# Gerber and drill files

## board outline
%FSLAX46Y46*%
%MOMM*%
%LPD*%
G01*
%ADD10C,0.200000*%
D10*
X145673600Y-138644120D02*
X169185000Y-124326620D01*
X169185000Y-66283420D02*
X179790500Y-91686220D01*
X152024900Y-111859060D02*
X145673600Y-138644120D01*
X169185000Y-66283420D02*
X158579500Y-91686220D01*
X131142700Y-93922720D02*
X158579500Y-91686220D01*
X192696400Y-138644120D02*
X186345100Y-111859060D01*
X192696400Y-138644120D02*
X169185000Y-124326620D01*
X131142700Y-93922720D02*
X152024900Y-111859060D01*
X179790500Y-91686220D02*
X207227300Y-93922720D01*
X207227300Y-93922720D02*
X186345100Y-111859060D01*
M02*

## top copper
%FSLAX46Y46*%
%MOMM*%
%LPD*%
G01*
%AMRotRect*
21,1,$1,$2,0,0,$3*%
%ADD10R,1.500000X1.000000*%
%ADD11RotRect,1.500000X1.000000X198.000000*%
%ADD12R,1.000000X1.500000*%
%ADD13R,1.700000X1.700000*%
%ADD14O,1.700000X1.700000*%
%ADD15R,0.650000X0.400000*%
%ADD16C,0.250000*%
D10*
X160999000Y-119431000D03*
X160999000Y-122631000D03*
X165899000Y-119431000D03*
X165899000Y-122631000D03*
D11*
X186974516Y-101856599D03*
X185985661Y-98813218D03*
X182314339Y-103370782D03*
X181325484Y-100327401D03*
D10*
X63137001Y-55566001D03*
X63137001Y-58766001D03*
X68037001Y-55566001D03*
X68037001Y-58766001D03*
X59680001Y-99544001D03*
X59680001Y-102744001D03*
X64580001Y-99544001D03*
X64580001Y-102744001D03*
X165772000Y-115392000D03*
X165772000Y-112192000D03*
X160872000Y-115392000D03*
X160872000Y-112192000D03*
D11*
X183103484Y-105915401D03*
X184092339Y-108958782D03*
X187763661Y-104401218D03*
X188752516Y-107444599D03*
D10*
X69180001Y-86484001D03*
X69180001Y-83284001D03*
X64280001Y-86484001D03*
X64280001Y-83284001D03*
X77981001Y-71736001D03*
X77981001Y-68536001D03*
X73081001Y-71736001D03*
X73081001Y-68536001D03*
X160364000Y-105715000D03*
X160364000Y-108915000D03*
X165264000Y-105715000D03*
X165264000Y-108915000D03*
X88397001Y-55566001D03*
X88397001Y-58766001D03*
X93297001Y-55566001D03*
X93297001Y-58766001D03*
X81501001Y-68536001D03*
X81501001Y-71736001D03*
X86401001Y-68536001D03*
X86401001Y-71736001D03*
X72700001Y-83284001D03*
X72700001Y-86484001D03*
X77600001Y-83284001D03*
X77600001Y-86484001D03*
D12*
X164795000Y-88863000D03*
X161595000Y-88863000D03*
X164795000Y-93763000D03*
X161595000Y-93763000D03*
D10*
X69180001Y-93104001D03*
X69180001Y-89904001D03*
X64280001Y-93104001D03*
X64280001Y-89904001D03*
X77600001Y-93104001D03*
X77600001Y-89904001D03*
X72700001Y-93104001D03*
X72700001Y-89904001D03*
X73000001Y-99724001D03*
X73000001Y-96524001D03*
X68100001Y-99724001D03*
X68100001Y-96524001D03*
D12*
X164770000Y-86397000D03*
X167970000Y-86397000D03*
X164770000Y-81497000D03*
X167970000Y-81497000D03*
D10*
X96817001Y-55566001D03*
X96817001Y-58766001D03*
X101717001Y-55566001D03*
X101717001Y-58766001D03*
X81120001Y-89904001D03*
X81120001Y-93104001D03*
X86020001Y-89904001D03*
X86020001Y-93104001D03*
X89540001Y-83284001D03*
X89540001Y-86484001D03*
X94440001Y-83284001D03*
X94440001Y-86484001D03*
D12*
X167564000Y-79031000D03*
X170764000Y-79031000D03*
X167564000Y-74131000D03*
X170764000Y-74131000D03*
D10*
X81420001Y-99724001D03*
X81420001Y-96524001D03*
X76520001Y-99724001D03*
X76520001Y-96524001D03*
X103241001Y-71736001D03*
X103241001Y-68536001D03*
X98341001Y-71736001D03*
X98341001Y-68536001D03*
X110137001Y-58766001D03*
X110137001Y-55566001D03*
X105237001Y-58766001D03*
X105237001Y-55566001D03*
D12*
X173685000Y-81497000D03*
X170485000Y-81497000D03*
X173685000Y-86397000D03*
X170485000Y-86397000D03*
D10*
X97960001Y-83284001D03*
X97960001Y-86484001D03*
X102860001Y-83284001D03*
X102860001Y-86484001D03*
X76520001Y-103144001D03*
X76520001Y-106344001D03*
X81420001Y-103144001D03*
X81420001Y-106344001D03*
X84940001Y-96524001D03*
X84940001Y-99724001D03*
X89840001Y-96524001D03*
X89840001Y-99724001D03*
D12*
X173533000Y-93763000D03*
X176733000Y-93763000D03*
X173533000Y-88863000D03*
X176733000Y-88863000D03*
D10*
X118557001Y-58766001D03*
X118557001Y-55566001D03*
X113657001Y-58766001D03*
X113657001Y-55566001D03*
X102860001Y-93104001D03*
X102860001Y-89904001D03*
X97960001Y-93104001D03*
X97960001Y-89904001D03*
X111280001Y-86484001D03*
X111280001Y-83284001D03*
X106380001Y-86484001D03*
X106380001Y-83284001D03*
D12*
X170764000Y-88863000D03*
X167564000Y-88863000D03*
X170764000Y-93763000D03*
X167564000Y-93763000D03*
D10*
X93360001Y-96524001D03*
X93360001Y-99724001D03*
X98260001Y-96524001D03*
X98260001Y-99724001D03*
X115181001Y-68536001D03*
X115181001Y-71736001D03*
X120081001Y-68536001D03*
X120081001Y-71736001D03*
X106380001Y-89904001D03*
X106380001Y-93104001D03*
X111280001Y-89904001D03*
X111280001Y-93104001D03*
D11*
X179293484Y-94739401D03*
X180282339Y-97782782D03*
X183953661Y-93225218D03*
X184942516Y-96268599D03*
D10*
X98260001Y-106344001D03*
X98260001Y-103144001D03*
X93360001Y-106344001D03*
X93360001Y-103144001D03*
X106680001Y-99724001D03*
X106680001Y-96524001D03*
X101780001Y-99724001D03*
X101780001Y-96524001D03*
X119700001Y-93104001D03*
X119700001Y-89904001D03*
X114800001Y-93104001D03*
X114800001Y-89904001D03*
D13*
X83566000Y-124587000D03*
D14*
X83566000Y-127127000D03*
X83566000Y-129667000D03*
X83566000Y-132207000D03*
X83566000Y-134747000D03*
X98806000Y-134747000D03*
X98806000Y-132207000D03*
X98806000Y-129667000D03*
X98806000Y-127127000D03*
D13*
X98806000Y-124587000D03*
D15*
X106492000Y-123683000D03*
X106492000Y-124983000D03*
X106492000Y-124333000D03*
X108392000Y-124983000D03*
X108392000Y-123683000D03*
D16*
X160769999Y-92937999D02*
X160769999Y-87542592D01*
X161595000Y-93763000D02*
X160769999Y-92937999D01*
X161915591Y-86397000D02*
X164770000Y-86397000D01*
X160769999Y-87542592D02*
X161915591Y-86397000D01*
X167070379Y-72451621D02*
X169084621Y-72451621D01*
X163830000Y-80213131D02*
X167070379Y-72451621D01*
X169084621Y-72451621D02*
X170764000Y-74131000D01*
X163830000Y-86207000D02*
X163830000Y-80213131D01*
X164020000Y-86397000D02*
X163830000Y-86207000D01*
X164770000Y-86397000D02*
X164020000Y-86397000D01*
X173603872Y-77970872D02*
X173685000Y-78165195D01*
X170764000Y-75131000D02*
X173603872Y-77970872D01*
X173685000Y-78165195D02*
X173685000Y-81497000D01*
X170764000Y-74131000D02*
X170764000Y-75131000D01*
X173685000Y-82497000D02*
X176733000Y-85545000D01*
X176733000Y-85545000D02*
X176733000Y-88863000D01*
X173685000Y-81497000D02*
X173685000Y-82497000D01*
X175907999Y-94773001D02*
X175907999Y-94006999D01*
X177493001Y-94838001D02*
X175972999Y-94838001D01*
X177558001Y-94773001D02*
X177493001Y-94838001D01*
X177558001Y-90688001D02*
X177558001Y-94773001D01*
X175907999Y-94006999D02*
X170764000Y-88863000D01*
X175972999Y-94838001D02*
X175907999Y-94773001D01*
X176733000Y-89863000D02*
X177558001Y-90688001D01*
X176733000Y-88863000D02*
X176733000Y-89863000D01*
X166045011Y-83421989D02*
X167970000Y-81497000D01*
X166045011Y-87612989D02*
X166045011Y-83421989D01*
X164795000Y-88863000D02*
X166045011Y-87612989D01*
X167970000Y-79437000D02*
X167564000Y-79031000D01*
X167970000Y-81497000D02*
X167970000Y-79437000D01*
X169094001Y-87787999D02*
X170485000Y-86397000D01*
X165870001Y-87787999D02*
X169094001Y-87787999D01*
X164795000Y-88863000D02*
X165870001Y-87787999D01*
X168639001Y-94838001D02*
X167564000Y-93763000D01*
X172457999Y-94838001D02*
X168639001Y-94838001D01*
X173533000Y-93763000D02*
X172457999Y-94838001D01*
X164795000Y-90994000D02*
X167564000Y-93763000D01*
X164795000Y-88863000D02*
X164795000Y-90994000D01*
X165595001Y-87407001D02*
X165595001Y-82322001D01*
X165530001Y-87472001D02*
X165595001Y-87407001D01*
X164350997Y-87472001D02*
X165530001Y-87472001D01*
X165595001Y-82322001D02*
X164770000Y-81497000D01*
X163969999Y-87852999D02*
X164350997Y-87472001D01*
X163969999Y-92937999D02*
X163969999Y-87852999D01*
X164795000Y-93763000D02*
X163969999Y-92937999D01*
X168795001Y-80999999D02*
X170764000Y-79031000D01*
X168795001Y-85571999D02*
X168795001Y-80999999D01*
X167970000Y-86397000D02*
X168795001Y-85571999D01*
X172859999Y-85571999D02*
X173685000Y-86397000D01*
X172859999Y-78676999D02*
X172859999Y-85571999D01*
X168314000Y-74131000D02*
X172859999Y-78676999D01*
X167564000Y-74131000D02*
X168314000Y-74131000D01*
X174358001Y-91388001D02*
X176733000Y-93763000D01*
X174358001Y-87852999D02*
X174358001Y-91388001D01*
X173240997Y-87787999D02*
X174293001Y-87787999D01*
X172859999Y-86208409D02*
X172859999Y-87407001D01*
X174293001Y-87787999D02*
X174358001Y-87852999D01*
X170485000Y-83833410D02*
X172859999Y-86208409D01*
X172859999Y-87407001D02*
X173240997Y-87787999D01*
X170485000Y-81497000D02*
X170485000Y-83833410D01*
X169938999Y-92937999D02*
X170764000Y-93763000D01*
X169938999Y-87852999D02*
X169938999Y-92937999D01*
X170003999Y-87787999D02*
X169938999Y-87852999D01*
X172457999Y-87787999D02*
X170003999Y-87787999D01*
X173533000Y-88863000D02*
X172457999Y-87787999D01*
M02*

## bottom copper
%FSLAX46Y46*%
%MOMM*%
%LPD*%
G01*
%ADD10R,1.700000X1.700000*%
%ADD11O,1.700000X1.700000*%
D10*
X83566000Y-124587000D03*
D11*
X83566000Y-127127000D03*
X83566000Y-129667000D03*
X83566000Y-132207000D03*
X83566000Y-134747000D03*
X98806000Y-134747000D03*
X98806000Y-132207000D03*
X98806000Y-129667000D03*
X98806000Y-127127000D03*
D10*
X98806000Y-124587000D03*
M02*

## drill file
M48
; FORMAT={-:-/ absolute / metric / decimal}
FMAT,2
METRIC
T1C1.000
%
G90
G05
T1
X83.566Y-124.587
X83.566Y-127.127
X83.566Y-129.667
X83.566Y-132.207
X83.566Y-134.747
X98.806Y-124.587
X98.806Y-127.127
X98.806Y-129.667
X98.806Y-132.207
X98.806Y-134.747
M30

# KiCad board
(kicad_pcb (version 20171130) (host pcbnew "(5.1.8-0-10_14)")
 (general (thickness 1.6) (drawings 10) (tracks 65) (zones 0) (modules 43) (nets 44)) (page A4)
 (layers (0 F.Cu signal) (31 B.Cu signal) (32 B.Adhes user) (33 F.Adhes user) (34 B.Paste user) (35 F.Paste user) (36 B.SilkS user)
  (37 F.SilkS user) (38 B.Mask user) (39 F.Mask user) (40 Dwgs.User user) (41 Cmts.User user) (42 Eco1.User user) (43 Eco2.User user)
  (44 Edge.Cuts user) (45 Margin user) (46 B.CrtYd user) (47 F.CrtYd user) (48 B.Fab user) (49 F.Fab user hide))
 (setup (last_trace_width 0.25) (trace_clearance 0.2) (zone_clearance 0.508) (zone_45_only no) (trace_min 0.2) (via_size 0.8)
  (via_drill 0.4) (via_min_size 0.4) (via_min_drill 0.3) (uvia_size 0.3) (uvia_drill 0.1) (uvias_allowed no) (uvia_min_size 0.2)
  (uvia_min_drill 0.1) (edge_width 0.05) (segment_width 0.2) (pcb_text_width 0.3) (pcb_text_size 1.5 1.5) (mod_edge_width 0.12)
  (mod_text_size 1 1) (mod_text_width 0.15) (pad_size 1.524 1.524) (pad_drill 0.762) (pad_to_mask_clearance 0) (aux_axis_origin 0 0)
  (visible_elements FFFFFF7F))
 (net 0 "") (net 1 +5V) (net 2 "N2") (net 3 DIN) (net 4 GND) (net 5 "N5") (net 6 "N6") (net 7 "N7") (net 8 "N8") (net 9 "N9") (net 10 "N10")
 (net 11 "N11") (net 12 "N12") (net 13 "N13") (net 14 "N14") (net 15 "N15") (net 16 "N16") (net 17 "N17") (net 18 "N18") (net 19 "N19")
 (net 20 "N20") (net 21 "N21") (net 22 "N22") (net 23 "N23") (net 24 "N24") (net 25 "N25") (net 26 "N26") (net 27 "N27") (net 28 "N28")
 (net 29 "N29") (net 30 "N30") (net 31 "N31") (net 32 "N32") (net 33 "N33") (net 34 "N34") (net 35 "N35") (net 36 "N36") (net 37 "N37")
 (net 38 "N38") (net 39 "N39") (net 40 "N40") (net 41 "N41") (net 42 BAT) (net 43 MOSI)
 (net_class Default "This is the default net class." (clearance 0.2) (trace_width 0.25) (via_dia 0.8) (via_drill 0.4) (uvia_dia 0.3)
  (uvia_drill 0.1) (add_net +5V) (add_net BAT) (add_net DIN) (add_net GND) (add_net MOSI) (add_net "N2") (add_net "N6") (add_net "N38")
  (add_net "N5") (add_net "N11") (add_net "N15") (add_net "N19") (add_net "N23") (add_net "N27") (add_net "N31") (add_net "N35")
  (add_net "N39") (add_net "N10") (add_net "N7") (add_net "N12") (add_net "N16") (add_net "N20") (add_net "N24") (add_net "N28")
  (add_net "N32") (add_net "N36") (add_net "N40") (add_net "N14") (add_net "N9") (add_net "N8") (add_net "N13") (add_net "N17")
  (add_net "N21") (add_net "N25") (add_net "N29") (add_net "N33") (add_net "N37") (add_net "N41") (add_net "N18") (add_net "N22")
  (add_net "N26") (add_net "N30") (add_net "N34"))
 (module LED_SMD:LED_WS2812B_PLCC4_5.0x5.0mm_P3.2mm (layer F.Cu) (at 163.449 121.031)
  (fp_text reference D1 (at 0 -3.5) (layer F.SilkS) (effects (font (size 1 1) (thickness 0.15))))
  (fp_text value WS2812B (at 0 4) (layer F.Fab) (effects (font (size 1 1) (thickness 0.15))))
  (pad 1 smd rect (at -2.45 -1.6) (size 1.5 1) (layers F.Cu F.Paste F.Mask) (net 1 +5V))
  (pad 2 smd rect (at -2.45 1.6) (size 1.5 1) (layers F.Cu F.Paste F.Mask) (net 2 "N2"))
  (pad 4 smd rect (at 2.45 -1.6) (size 1.5 1) (layers F.Cu F.Paste F.Mask) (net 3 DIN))
  (pad 3 smd rect (at 2.45 1.6) (size 1.5 1) (layers F.Cu F.Paste F.Mask) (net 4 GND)))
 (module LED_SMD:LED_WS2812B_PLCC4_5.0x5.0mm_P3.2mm (layer F.Cu) (at 184.15 101.092 198)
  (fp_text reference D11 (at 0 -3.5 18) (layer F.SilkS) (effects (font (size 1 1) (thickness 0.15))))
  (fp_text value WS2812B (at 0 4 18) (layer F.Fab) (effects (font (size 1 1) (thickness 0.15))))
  (pad 1 smd rect (at -2.45 -1.6 198) (size 1.5 1) (layers F.Cu F.Paste F.Mask) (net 1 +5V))
  (pad 2 smd rect (at -2.45 1.6 198) (size 1.5 1) (layers F.Cu F.Paste F.Mask) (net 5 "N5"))
  (pad 4 smd rect (at 2.45 -1.6 198) (size 1.5 1) (layers F.Cu F.Paste F.Mask) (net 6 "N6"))
  (pad 3 smd rect (at 2.45 1.6 198) (size 1.5 1) (layers F.Cu F.Paste F.Mask) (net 4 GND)))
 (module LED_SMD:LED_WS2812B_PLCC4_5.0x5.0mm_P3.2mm (layer F.Cu) (at 65.587001 57.166001)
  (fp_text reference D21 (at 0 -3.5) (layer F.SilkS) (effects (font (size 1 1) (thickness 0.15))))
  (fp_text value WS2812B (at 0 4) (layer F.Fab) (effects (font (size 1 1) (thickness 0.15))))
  (pad 1 smd rect (at -2.45 -1.6) (size 1.5 1) (layers F.Cu F.Paste F.Mask) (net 1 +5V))
  (pad 2 smd rect (at -2.45 1.6) (size 1.5 1) (layers F.Cu F.Paste F.Mask) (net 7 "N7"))
  (pad 4 smd rect (at 2.45 -1.6) (size 1.5 1) (layers F.Cu F.Paste F.Mask))
  (pad 3 smd rect (at 2.45 1.6) (size 1.5 1) (layers F.Cu F.Paste F.Mask) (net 4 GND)))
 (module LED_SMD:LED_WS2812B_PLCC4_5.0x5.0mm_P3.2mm (layer F.Cu) (at 62.130001 101.144001)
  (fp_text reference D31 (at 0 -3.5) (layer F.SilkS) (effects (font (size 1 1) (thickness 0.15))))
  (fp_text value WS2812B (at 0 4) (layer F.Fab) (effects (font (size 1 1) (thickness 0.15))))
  (pad 1 smd rect (at -2.45 -1.6) (size 1.5 1) (layers F.Cu F.Paste F.Mask) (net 1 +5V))
  (pad 2 smd rect (at -2.45 1.6) (size 1.5 1) (layers F.Cu F.Paste F.Mask) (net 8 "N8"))
  (pad 4 smd rect (at 2.45 -1.6) (size 1.5 1) (layers F.Cu F.Paste F.Mask) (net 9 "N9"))
  (pad 3 smd rect (at 2.45 1.6) (size 1.5 1) (layers F.Cu F.Paste F.Mask) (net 4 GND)))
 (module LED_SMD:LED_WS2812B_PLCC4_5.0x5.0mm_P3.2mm (layer F.Cu) (at 163.322 113.792)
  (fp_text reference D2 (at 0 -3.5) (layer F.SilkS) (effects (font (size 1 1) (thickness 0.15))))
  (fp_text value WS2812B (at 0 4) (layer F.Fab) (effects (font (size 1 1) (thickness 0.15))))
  (pad 3 smd rect (at 2.45 1.6) (size 1.5 1) (layers F.Cu F.Paste F.Mask) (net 4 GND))
  (pad 4 smd rect (at 2.45 -1.6) (size 1.5 1) (layers F.Cu F.Paste F.Mask) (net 2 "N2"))
  (pad 2 smd rect (at -2.45 1.6) (size 1.5 1) (layers F.Cu F.Paste F.Mask) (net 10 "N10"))
  (pad 1 smd rect (at -2.45 -1.6) (size 1.5 1) (layers F.Cu F.Paste F.Mask) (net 1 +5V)))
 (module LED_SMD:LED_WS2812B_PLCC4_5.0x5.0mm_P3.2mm (layer F.Cu) (at 185.928 106.68 198)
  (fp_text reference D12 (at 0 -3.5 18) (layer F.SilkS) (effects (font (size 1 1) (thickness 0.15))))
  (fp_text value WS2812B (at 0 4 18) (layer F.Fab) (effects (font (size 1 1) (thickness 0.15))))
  (pad 3 smd rect (at 2.45 1.6 198) (size 1.5 1) (layers F.Cu F.Paste F.Mask) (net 4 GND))
  (pad 4 smd rect (at 2.45 -1.6 198) (size 1.5 1) (layers F.Cu F.Paste F.Mask) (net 5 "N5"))
  (pad 2 smd rect (at -2.45 1.6 198) (size 1.5 1) (layers F.Cu F.Paste F.Mask) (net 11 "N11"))
  (pad 1 smd rect (at -2.45 -1.6 198) (size 1.5 1) (layers F.Cu F.Paste F.Mask) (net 1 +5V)))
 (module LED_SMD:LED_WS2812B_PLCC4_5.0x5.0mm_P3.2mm (layer F.Cu) (at 66.730001 84.884001)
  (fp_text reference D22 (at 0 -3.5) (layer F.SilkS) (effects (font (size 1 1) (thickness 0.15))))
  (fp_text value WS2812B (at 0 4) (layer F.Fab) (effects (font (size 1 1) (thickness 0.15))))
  (pad 3 smd rect (at 2.45 1.6) (size 1.5 1) (layers F.Cu F.Paste F.Mask) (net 4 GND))
  (pad 4 smd rect (at 2.45 -1.6) (size 1.5 1) (layers F.Cu F.Paste F.Mask) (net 7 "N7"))
  (pad 2 smd rect (at -2.45 1.6) (size 1.5 1) (layers F.Cu F.Paste F.Mask) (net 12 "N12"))
  (pad 1 smd rect (at -2.45 -1.6) (size 1.5 1) (layers F.Cu F.Paste F.Mask) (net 1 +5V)))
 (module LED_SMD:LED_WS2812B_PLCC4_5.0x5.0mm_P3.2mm (layer F.Cu) (at 75.531001 70.136001)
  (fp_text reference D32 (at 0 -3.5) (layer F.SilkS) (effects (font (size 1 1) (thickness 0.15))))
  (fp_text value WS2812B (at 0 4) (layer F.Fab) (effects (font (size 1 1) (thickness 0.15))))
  (pad 3 smd rect (at 2.45 1.6) (size 1.5 1) (layers F.Cu F.Paste F.Mask) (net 4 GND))
  (pad 4 smd rect (at 2.45 -1.6) (size 1.5 1) (layers F.Cu F.Paste F.Mask) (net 8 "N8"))
  (pad 2 smd rect (at -2.45 1.6) (size 1.5 1) (layers F.Cu F.Paste F.Mask) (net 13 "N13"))
  (pad 1 smd rect (at -2.45 -1.6) (size 1.5 1) (layers F.Cu F.Paste F.Mask) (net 1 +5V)))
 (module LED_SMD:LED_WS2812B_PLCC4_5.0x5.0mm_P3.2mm (layer F.Cu) (at 162.814 107.315)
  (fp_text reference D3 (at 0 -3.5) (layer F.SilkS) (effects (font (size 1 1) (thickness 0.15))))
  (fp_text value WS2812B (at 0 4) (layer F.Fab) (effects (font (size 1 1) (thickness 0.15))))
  (pad 1 smd rect (at -2.45 -1.6) (size 1.5 1) (layers F.Cu F.Paste F.Mask) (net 1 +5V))
  (pad 2 smd rect (at -2.45 1.6) (size 1.5 1) (layers F.Cu F.Paste F.Mask) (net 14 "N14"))
  (pad 4 smd rect (at 2.45 -1.6) (size 1.5 1) (layers F.Cu F.Paste F.Mask) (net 10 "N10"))
  (pad 3 smd rect (at 2.45 1.6) (size 1.5 1) (layers F.Cu F.Paste F.Mask) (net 4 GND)))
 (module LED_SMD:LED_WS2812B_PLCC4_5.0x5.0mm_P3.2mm (layer F.Cu) (at 90.847001 57.166001)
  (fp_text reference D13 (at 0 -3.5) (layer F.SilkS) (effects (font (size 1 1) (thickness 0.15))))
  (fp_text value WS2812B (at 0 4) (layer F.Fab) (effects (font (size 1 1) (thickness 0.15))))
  (pad 1 smd rect (at -2.45 -1.6) (size 1.5 1) (layers F.Cu F.Paste F.Mask) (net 1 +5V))
  (pad 2 smd rect (at -2.45 1.6) (size 1.5 1) (layers F.Cu F.Paste F.Mask) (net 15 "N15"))
  (pad 4 smd rect (at 2.45 -1.6) (size 1.5 1) (layers F.Cu F.Paste F.Mask) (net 11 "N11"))
  (pad 3 smd rect (at 2.45 1.6) (size 1.5 1) (layers F.Cu F.Paste F.Mask) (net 4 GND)))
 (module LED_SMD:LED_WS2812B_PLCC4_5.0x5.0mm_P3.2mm (layer F.Cu) (at 83.951001 70.136001)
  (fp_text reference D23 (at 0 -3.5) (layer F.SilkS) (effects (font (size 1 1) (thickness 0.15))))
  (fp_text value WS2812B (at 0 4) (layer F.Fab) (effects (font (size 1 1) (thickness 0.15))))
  (pad 1 smd rect (at -2.45 -1.6) (size 1.5 1) (layers F.Cu F.Paste F.Mask) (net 1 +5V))
  (pad 2 smd rect (at -2.45 1.6) (size 1.5 1) (layers F.Cu F.Paste F.Mask) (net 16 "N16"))
  (pad 4 smd rect (at 2.45 -1.6) (size 1.5 1) (layers F.Cu F.Paste F.Mask) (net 12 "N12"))
  (pad 3 smd rect (at 2.45 1.6) (size 1.5 1) (layers F.Cu F.Paste F.Mask) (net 4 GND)))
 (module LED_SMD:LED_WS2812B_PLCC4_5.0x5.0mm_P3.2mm (layer F.Cu) (at 75.150001 84.884001)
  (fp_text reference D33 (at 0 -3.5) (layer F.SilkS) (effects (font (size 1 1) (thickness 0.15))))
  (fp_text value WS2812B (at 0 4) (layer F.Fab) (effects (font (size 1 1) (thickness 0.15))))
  (pad 1 smd rect (at -2.45 -1.6) (size 1.5 1) (layers F.Cu F.Paste F.Mask) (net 1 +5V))
  (pad 2 smd rect (at -2.45 1.6) (size 1.5 1) (layers F.Cu F.Paste F.Mask) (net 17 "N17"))
  (pad 4 smd rect (at 2.45 -1.6) (size 1.5 1) (layers F.Cu F.Paste F.Mask) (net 13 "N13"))
  (pad 3 smd rect (at 2.45 1.6) (size 1.5 1) (layers F.Cu F.Paste F.Mask) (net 4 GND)))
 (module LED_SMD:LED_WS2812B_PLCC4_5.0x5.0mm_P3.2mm (layer F.Cu) (at 163.195 91.313 90)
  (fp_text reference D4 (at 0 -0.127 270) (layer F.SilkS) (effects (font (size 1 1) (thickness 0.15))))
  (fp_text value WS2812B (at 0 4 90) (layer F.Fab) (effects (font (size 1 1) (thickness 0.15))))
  (pad 3 smd rect (at 2.45 1.6 90) (size 1.5 1) (layers F.Cu F.Paste F.Mask) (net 4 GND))
  (pad 4 smd rect (at 2.45 -1.6 90) (size 1.5 1) (layers F.Cu F.Paste F.Mask) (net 14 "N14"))
  (pad 2 smd rect (at -2.45 1.6 90) (size 1.5 1) (layers F.Cu F.Paste F.Mask) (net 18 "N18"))
  (pad 1 smd rect (at -2.45 -1.6 90) (size 1.5 1) (layers F.Cu F.Paste F.Mask) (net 1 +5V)))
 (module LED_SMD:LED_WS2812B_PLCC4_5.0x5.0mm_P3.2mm (layer F.Cu) (at 66.730001 91.504001)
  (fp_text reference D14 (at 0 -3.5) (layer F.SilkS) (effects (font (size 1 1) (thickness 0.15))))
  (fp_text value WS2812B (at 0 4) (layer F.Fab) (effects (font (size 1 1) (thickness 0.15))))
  (pad 3 smd rect (at 2.45 1.6) (size 1.5 1) (layers F.Cu F.Paste F.Mask) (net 4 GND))
  (pad 4 smd rect (at 2.45 -1.6) (size 1.5 1) (layers F.Cu F.Paste F.Mask) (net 15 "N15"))
  (pad 2 smd rect (at -2.45 1.6) (size 1.5 1) (layers F.Cu F.Paste F.Mask) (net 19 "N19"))
  (pad 1 smd rect (at -2.45 -1.6) (size 1.5 1) (layers F.Cu F.Paste F.Mask) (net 1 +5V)))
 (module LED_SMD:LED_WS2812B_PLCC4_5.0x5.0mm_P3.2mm (layer F.Cu) (at 75.150001 91.504001)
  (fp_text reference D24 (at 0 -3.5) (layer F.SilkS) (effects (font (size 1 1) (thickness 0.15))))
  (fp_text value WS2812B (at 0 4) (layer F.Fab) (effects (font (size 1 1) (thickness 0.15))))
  (pad 3 smd rect (at 2.45 1.6) (size 1.5 1) (layers F.Cu F.Paste F.Mask) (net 4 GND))
  (pad 4 smd rect (at 2.45 -1.6) (size 1.5 1) (layers F.Cu F.Paste F.Mask) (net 16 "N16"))
  (pad 2 smd rect (at -2.45 1.6) (size 1.5 1) (layers F.Cu F.Paste F.Mask) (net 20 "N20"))
  (pad 1 smd rect (at -2.45 -1.6) (size 1.5 1) (layers F.Cu F.Paste F.Mask) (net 1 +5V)))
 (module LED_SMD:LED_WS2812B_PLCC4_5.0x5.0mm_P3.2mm (layer F.Cu) (at 70.550001 98.124001)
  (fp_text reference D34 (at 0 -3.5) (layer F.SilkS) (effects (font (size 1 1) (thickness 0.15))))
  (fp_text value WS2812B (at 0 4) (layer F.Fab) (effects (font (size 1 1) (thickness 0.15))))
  (pad 3 smd rect (at 2.45 1.6) (size 1.5 1) (layers F.Cu F.Paste F.Mask) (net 4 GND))
  (pad 4 smd rect (at 2.45 -1.6) (size 1.5 1) (layers F.Cu F.Paste F.Mask) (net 17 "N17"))
  (pad 2 smd rect (at -2.45 1.6) (size 1.5 1) (layers F.Cu F.Paste F.Mask) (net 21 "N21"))
  (pad 1 smd rect (at -2.45 -1.6) (size 1.5 1) (layers F.Cu F.Paste F.Mask) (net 1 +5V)))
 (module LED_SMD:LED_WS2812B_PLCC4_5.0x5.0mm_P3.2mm (layer F.Cu) (at 166.37 83.947 90)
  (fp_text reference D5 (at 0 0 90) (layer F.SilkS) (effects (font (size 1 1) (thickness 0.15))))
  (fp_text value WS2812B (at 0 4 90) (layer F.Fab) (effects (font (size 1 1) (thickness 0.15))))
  (pad 1 smd rect (at -2.45 -1.6 90) (size 1.5 1) (layers F.Cu F.Paste F.Mask) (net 1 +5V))
  (pad 2 smd rect (at -2.45 1.6 90) (size 1.5 1) (layers F.Cu F.Paste F.Mask) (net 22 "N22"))
  (pad 4 smd rect (at 2.45 -1.6 90) (size 1.5 1) (layers F.Cu F.Paste F.Mask) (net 18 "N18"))
  (pad 3 smd rect (at 2.45 1.6 90) (size 1.5 1) (layers F.Cu F.Paste F.Mask) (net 4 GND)))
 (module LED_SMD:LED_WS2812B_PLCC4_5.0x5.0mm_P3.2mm (layer F.Cu) (at 99.267001 57.166001)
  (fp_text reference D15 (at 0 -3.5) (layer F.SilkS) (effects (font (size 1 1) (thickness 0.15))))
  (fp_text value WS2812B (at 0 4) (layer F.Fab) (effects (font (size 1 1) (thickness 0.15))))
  (pad 1 smd rect (at -2.45 -1.6) (size 1.5 1) (layers F.Cu F.Paste F.Mask) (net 1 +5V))
  (pad 2 smd rect (at -2.45 1.6) (size 1.5 1) (layers F.Cu F.Paste F.Mask) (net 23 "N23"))
  (pad 4 smd rect (at 2.45 -1.6) (size 1.5 1) (layers F.Cu F.Paste F.Mask) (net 19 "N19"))
  (pad 3 smd rect (at 2.45 1.6) (size 1.5 1) (layers F.Cu F.Paste F.Mask) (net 4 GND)))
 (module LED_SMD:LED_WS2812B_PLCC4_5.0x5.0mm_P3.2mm (layer F.Cu) (at 83.570001 91.504001)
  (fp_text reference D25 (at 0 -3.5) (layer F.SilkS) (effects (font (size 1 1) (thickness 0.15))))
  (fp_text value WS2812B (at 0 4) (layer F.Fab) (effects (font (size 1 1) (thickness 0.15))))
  (pad 1 smd rect (at -2.45 -1.6) (size 1.5 1) (layers F.Cu F.Paste F.Mask) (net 1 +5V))
  (pad 2 smd rect (at -2.45 1.6) (size 1.5 1) (layers F.Cu F.Paste F.Mask) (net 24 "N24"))
  (pad 4 smd rect (at 2.45 -1.6) (size 1.5 1) (layers F.Cu F.Paste F.Mask) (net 20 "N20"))
  (pad 3 smd rect (at 2.45 1.6) (size 1.5 1) (layers F.Cu F.Paste F.Mask) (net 4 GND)))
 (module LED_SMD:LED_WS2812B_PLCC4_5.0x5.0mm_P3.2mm (layer F.Cu) (at 91.990001 84.884001)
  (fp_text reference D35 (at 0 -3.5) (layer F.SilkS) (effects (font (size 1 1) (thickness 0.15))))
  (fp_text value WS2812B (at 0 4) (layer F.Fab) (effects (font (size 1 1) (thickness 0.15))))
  (pad 1 smd rect (at -2.45 -1.6) (size 1.5 1) (layers F.Cu F.Paste F.Mask) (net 1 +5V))
  (pad 2 smd rect (at -2.45 1.6) (size 1.5 1) (layers F.Cu F.Paste F.Mask) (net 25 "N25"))
  (pad 4 smd rect (at 2.45 -1.6) (size 1.5 1) (layers F.Cu F.Paste F.Mask) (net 21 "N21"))
  (pad 3 smd rect (at 2.45 1.6) (size 1.5 1) (layers F.Cu F.Paste F.Mask) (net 4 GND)))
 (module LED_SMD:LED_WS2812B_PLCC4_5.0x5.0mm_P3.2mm (layer F.Cu) (at 169.164 76.581 270)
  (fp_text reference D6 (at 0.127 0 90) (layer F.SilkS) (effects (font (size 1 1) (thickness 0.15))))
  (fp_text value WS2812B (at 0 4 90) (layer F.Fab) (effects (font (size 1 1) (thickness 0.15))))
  (pad 3 smd rect (at 2.45 1.6 270) (size 1.5 1) (layers F.Cu F.Paste F.Mask) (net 4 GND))
  (pad 4 smd rect (at 2.45 -1.6 270) (size 1.5 1) (layers F.Cu F.Paste F.Mask) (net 22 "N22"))
  (pad 2 smd rect (at -2.45 1.6 270) (size 1.5 1) (layers F.Cu F.Paste F.Mask) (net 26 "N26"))
  (pad 1 smd rect (at -2.45 -1.6 270) (size 1.5 1) (layers F.Cu F.Paste F.Mask) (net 1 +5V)))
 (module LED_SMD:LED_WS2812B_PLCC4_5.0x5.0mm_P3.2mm (layer F.Cu) (at 78.970001 98.124001)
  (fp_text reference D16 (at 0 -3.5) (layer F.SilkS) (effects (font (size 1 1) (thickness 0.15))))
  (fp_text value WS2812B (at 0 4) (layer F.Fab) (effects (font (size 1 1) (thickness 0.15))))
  (pad 3 smd rect (at 2.45 1.6) (size 1.5 1) (layers F.Cu F.Paste F.Mask) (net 4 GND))
  (pad 4 smd rect (at 2.45 -1.6) (size 1.5 1) (layers F.Cu F.Paste F.Mask) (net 23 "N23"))
  (pad 2 smd rect (at -2.45 1.6) (size 1.5 1) (layers F.Cu F.Paste F.Mask) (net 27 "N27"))
  (pad 1 smd rect (at -2.45 -1.6) (size 1.5 1) (layers F.Cu F.Paste F.Mask) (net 1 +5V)))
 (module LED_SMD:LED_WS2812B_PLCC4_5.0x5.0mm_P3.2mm (layer F.Cu) (at 100.791001 70.136001)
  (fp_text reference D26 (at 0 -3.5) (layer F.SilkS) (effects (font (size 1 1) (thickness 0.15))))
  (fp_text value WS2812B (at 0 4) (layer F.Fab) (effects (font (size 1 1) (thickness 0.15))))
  (pad 3 smd rect (at 2.45 1.6) (size 1.5 1) (layers F.Cu F.Paste F.Mask) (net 4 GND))
  (pad 4 smd rect (at 2.45 -1.6) (size 1.5 1) (layers F.Cu F.Paste F.Mask) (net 24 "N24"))
  (pad 2 smd rect (at -2.45 1.6) (size 1.5 1) (layers F.Cu F.Paste F.Mask) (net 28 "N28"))
  (pad 1 smd rect (at -2.45 -1.6) (size 1.5 1) (layers F.Cu F.Paste F.Mask) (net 1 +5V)))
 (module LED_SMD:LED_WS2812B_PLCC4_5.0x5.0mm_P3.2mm (layer F.Cu) (at 107.687001 57.166001)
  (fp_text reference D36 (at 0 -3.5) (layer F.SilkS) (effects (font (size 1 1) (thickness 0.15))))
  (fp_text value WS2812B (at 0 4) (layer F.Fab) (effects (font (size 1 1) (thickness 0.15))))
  (pad 3 smd rect (at 2.45 1.6) (size 1.5 1) (layers F.Cu F.Paste F.Mask) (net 4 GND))
  (pad 4 smd rect (at 2.45 -1.6) (size 1.5 1) (layers F.Cu F.Paste F.Mask) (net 25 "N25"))
  (pad 2 smd rect (at -2.45 1.6) (size 1.5 1) (layers F.Cu F.Paste F.Mask) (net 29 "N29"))
  (pad 1 smd rect (at -2.45 -1.6) (size 1.5 1) (layers F.Cu F.Paste F.Mask) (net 1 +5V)))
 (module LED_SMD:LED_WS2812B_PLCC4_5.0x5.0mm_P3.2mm (layer F.Cu) (at 172.085 83.947 270)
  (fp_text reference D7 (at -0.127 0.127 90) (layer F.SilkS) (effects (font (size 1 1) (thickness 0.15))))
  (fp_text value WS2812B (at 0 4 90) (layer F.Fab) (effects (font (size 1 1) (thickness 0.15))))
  (pad 1 smd rect (at -2.45 -1.6 270) (size 1.5 1) (layers F.Cu F.Paste F.Mask) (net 1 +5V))
  (pad 2 smd rect (at -2.45 1.6 270) (size 1.5 1) (layers F.Cu F.Paste F.Mask) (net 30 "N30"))
  (pad 4 smd rect (at 2.45 -1.6 270) (size 1.5 1) (layers F.Cu F.Paste F.Mask) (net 26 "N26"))
  (pad 3 smd rect (at 2.45 1.6 270) (size 1.5 1) (layers F.Cu F.Paste F.Mask) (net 4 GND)))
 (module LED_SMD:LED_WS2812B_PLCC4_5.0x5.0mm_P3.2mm (layer F.Cu) (at 100.410001 84.884001)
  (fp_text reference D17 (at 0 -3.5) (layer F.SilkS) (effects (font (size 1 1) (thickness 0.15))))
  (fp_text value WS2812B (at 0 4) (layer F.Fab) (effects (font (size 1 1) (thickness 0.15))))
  (pad 1 smd rect (at -2.45 -1.6) (size 1.5 1) (layers F.Cu F.Paste F.Mask) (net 1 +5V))
  (pad 2 smd rect (at -2.45 1.6) (size 1.5 1) (layers F.Cu F.Paste F.Mask) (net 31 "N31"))
  (pad 4 smd rect (at 2.45 -1.6) (size 1.5 1) (layers F.Cu F.Paste F.Mask) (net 27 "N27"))
  (pad 3 smd rect (at 2.45 1.6) (size 1.5 1) (layers F.Cu F.Paste F.Mask) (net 4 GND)))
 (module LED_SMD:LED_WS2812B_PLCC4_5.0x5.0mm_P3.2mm (layer F.Cu) (at 78.970001 104.744001)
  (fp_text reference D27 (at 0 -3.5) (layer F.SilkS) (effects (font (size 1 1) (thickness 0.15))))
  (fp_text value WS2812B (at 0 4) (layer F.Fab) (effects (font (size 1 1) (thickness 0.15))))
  (pad 1 smd rect (at -2.45 -1.6) (size 1.5 1) (layers F.Cu F.Paste F.Mask) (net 1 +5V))
  (pad 2 smd rect (at -2.45 1.6) (size 1.5 1) (layers F.Cu F.Paste F.Mask) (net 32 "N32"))
  (pad 4 smd rect (at 2.45 -1.6) (size 1.5 1) (layers F.Cu F.Paste F.Mask) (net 28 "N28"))
  (pad 3 smd rect (at 2.45 1.6) (size 1.5 1) (layers F.Cu F.Paste F.Mask) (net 4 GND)))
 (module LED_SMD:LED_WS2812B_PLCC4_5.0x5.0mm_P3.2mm (layer F.Cu) (at 87.390001 98.124001)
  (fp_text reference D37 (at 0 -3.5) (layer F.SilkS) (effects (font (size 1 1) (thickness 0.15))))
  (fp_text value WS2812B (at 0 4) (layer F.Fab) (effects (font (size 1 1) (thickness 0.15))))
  (pad 1 smd rect (at -2.45 -1.6) (size 1.5 1) (layers F.Cu F.Paste F.Mask) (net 1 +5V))
  (pad 2 smd rect (at -2.45 1.6) (size 1.5 1) (layers F.Cu F.Paste F.Mask) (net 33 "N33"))
  (pad 4 smd rect (at 2.45 -1.6) (size 1.5 1) (layers F.Cu F.Paste F.Mask) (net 29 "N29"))
  (pad 3 smd rect (at 2.45 1.6) (size 1.5 1) (layers F.Cu F.Paste F.Mask) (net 4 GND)))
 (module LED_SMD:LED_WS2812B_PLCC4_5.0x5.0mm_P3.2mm (layer F.Cu) (at 175.133 91.313 270)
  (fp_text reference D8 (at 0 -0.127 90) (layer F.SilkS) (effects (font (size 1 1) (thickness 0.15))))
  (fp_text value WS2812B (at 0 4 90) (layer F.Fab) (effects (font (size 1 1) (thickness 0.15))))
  (pad 3 smd rect (at 2.45 1.6 270) (size 1.5 1) (layers F.Cu F.Paste F.Mask) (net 4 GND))
  (pad 4 smd rect (at 2.45 -1.6 270) (size 1.5 1) (layers F.Cu F.Paste F.Mask) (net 30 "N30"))
  (pad 2 smd rect (at -2.45 1.6 270) (size 1.5 1) (layers F.Cu F.Paste F.Mask) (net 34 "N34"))
  (pad 1 smd rect (at -2.45 -1.6 270) (size 1.5 1) (layers F.Cu F.Paste F.Mask) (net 1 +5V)))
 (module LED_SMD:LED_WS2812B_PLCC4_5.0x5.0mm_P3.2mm (layer F.Cu) (at 116.107001 57.166001)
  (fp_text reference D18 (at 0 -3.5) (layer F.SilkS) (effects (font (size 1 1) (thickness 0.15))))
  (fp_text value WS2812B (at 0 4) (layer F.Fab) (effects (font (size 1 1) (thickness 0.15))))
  (pad 3 smd rect (at 2.45 1.6) (size 1.5 1) (layers F.Cu F.Paste F.Mask) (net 4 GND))
  (pad 4 smd rect (at 2.45 -1.6) (size 1.5 1) (layers F.Cu F.Paste F.Mask) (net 31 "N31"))
  (pad 2 smd rect (at -2.45 1.6) (size 1.5 1) (layers F.Cu F.Paste F.Mask) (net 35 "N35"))
  (pad 1 smd rect (at -2.45 -1.6) (size 1.5 1) (layers F.Cu F.Paste F.Mask) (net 1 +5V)))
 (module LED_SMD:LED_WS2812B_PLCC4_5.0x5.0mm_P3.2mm (layer F.Cu) (at 100.410001 91.504001)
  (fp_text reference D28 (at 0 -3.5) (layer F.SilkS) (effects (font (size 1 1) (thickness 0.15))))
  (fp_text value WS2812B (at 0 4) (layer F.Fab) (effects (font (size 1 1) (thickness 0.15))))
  (pad 3 smd rect (at 2.45 1.6) (size 1.5 1) (layers F.Cu F.Paste F.Mask) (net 4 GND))
  (pad 4 smd rect (at 2.45 -1.6) (size 1.5 1) (layers F.Cu F.Paste F.Mask) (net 32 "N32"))
  (pad 2 smd rect (at -2.45 1.6) (size 1.5 1) (layers F.Cu F.Paste F.Mask) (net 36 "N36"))
  (pad 1 smd rect (at -2.45 -1.6) (size 1.5 1) (layers F.Cu F.Paste F.Mask) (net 1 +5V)))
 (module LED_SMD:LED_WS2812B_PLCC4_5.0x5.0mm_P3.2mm (layer F.Cu) (at 108.830001 84.884001)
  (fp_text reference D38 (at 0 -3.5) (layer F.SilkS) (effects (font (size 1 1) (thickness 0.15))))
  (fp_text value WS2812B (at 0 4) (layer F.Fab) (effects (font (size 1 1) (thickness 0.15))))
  (pad 3 smd rect (at 2.45 1.6) (size 1.5 1) (layers F.Cu F.Paste F.Mask) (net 4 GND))
  (pad 4 smd rect (at 2.45 -1.6) (size 1.5 1) (layers F.Cu F.Paste F.Mask) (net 33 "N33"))
  (pad 2 smd rect (at -2.45 1.6) (size 1.5 1) (layers F.Cu F.Paste F.Mask) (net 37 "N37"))
  (pad 1 smd rect (at -2.45 -1.6) (size 1.5 1) (layers F.Cu F.Paste F.Mask) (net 1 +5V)))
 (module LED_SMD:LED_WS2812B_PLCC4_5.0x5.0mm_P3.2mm (layer F.Cu) (at 169.164 91.313 270)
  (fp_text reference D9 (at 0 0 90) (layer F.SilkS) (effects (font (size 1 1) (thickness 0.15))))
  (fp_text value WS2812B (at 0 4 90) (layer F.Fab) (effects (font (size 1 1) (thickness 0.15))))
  (pad 1 smd rect (at -2.45 -1.6 270) (size 1.5 1) (layers F.Cu F.Paste F.Mask) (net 1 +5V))
  (pad 2 smd rect (at -2.45 1.6 270) (size 1.5 1) (layers F.Cu F.Paste F.Mask) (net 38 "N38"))
  (pad 4 smd rect (at 2.45 -1.6 270) (size 1.5 1) (layers F.Cu F.Paste F.Mask) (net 34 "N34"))
  (pad 3 smd rect (at 2.45 1.6 270) (size 1.5 1) (layers F.Cu F.Paste F.Mask) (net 4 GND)))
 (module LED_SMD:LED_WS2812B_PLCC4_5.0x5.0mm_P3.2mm (layer F.Cu) (at 95.810001 98.124001)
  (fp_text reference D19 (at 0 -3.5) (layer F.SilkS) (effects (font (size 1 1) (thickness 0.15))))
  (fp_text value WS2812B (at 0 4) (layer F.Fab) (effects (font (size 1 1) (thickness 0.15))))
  (pad 1 smd rect (at -2.45 -1.6) (size 1.5 1) (layers F.Cu F.Paste F.Mask) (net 1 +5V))
  (pad 2 smd rect (at -2.45 1.6) (size 1.5 1) (layers F.Cu F.Paste F.Mask) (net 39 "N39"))
  (pad 4 smd rect (at 2.45 -1.6) (size 1.5 1) (layers F.Cu F.Paste F.Mask) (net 35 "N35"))
  (pad 3 smd rect (at 2.45 1.6) (size 1.5 1) (layers F.Cu F.Paste F.Mask) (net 4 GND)))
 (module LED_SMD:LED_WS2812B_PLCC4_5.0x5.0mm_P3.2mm (layer F.Cu) (at 117.631001 70.136001)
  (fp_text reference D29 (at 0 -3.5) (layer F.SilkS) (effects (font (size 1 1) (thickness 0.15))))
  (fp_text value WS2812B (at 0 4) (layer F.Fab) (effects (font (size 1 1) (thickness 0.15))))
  (pad 1 smd rect (at -2.45 -1.6) (size 1.5 1) (layers F.Cu F.Paste F.Mask) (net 1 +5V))
  (pad 2 smd rect (at -2.45 1.6) (size 1.5 1) (layers F.Cu F.Paste F.Mask) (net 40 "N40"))
  (pad 4 smd rect (at 2.45 -1.6) (size 1.5 1) (layers F.Cu F.Paste F.Mask) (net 36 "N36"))
  (pad 3 smd rect (at 2.45 1.6) (size 1.5 1) (layers F.Cu F.Paste F.Mask) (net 4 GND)))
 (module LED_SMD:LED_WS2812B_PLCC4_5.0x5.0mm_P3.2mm (layer F.Cu) (at 108.830001 91.504001)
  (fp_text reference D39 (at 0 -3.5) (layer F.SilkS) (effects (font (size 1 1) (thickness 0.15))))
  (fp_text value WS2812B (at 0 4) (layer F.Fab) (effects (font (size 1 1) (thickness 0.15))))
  (pad 1 smd rect (at -2.45 -1.6) (size 1.5 1) (layers F.Cu F.Paste F.Mask) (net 1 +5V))
  (pad 2 smd rect (at -2.45 1.6) (size 1.5 1) (layers F.Cu F.Paste F.Mask) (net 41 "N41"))
  (pad 4 smd rect (at 2.45 -1.6) (size 1.5 1) (layers F.Cu F.Paste F.Mask) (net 37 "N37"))
  (pad 3 smd rect (at 2.45 1.6) (size 1.5 1) (layers F.Cu F.Paste F.Mask) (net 4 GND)))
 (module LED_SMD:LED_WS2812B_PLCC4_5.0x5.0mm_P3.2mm (layer F.Cu) (at 182.118 95.504 198)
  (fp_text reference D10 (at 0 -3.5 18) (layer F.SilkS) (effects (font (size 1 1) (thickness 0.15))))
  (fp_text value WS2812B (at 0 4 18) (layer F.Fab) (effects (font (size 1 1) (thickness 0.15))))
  (pad 3 smd rect (at 2.45 1.6 198) (size 1.5 1) (layers F.Cu F.Paste F.Mask) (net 4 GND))
  (pad 4 smd rect (at 2.45 -1.6 198) (size 1.5 1) (layers F.Cu F.Paste F.Mask) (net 38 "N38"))
  (pad 2 smd rect (at -2.45 1.6 198) (size 1.5 1) (layers F.Cu F.Paste F.Mask) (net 6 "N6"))
  (pad 1 smd rect (at -2.45 -1.6 198) (size 1.5 1) (layers F.Cu F.Paste F.Mask) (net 1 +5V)))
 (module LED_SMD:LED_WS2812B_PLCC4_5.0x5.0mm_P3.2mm (layer F.Cu) (at 95.810001 104.744001)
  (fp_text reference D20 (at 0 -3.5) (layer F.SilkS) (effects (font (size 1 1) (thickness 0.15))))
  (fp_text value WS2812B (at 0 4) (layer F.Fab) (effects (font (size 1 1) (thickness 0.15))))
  (pad 3 smd rect (at 2.45 1.6) (size 1.5 1) (layers F.Cu F.Paste F.Mask) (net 4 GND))
  (pad 4 smd rect (at 2.45 -1.6) (size 1.5 1) (layers F.Cu F.Paste F.Mask) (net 39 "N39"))
  (pad 2 smd rect (at -2.45 1.6) (size 1.5 1) (layers F.Cu F.Paste F.Mask))
  (pad 1 smd rect (at -2.45 -1.6) (size 1.5 1) (layers F.Cu F.Paste F.Mask) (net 1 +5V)))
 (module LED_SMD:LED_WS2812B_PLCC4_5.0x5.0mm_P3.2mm (layer F.Cu) (at 104.230001 98.124001)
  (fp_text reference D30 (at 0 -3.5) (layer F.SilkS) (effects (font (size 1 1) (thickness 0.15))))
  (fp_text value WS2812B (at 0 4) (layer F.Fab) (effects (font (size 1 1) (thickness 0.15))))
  (pad 3 smd rect (at 2.45 1.6) (size 1.5 1) (layers F.Cu F.Paste F.Mask) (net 4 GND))
  (pad 4 smd rect (at 2.45 -1.6) (size 1.5 1) (layers F.Cu F.Paste F.Mask) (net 40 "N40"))
  (pad 2 smd rect (at -2.45 1.6) (size 1.5 1) (layers F.Cu F.Paste F.Mask) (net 9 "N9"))
  (pad 1 smd rect (at -2.45 -1.6) (size 1.5 1) (layers F.Cu F.Paste F.Mask) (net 1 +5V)))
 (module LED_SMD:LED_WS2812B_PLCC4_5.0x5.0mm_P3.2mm (layer F.Cu) (at 117.250001 91.504001)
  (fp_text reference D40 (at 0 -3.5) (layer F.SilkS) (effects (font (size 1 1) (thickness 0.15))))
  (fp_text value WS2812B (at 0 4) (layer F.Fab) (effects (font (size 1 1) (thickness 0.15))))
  (pad 3 smd rect (at 2.45 1.6) (size 1.5 1) (layers F.Cu F.Paste F.Mask) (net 4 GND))
  (pad 4 smd rect (at 2.45 -1.6) (size 1.5 1) (layers F.Cu F.Paste F.Mask) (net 41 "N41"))
  (pad 2 smd rect (at -2.45 1.6) (size 1.5 1) (layers F.Cu F.Paste F.Mask))
  (pad 1 smd rect (at -2.45 -1.6) (size 1.5 1) (layers F.Cu F.Paste F.Mask) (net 1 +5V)))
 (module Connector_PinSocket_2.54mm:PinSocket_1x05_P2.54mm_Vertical (layer F.Cu) (at 83.566 124.587)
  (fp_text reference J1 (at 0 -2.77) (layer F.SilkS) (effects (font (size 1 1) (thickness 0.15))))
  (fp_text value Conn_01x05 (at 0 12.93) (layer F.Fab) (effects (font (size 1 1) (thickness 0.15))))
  (pad 1 thru_hole rect (at 0 0) (size 1.7 1.7) (drill 1) (layers *.Cu *.Mask) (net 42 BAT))
  (pad 2 thru_hole oval (at 0 2.54) (size 1.7 1.7) (drill 1) (layers *.Cu *.Mask) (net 4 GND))
  (pad 3 thru_hole oval (at 0 5.08) (size 1.7 1.7) (drill 1) (layers *.Cu *.Mask) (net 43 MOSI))
  (pad 4 thru_hole oval (at 0 7.62) (size 1.7 1.7) (drill 1) (layers *.Cu *.Mask))
  (pad 5 thru_hole oval (at 0 10.16) (size 1.7 1.7) (drill 1) (layers *.Cu *.Mask)))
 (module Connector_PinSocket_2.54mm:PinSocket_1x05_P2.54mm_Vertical (layer F.Cu) (at 98.806 124.587)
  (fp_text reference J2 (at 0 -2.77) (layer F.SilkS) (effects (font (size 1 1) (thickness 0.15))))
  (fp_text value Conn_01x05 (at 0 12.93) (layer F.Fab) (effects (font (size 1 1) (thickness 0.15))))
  (pad 5 thru_hole oval (at 0 10.16) (size 1.7 1.7) (drill 1) (layers *.Cu *.Mask))
  (pad 4 thru_hole oval (at 0 7.62) (size 1.7 1.7) (drill 1) (layers *.Cu *.Mask))
  (pad 3 thru_hole oval (at 0 5.08) (size 1.7 1.7) (drill 1) (layers *.Cu *.Mask))
  (pad 2 thru_hole oval (at 0 2.54) (size 1.7 1.7) (drill 1) (layers *.Cu *.Mask))
  (pad 1 thru_hole rect (at 0 0) (size 1.7 1.7) (drill 1) (layers *.Cu *.Mask)))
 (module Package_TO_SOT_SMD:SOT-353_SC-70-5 (layer F.Cu) (at 107.442 124.333)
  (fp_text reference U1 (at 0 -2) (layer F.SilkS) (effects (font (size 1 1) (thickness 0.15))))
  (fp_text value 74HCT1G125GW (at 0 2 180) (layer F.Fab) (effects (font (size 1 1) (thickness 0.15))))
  (pad 1 smd rect (at -0.95 -0.65) (size 0.65 0.4) (layers F.Cu F.Paste F.Mask) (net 4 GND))
  (pad 3 smd rect (at -0.95 0.65) (size 0.65 0.4) (layers F.Cu F.Paste F.Mask) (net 4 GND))
  (pad 2 smd rect (at -0.95 0) (size 0.65 0.4) (layers F.Cu F.Paste F.Mask) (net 43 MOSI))
  (pad 4 smd rect (at 0.95 0.65) (size 0.65 0.4) (layers F.Cu F.Paste F.Mask) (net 3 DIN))
  (pad 5 smd rect (at 0.95 -0.65) (size 0.65 0.4) (layers F.Cu F.Paste F.Mask) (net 42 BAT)))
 (gr_line (start 145.6736 138.64412) (end 169.185 124.32662) (layer Edge.Cuts) (width 0.2))
 (gr_line (start 169.185 66.28342) (end 179.7905 91.68622) (layer Edge.Cuts) (width 0.2))
 (gr_line (start 152.0249 111.85906) (end 145.6736 138.64412) (layer Edge.Cuts) (width 0.2))
 (gr_line (start 169.185 66.28342) (end 158.5795 91.68622) (layer Edge.Cuts) (width 0.2))
 (gr_line (start 131.1427 93.92272) (end 158.5795 91.68622) (layer Edge.Cuts) (width 0.2))
 (gr_line (start 192.6964 138.64412) (end 186.3451 111.85906) (layer Edge.Cuts) (width 0.2))
 (gr_line (start 192.6964 138.64412) (end 169.185 124.32662) (layer Edge.Cuts) (width 0.2))
 (gr_line (start 131.1427 93.92272) (end 152.0249 111.85906) (layer Edge.Cuts) (width 0.2))
 (gr_line (start 179.7905 91.68622) (end 207.2273 93.92272) (layer Edge.Cuts) (width 0.2))
 (gr_line (start 207.2273 93.92272) (end 186.3451 111.85906) (layer Edge.Cuts) (width 0.2))
 (segment (start 160.769999 92.937999) (end 160.769999 87.542592) (width 0.25) (layer F.Cu) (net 1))
 (segment (start 161.595 93.763) (end 160.769999 92.937999) (width 0.25) (layer F.Cu) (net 1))
 (segment (start 161.915591 86.397) (end 164.77 86.397) (width 0.25) (layer F.Cu) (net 1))
 (segment (start 160.769999 87.542592) (end 161.915591 86.397) (width 0.25) (layer F.Cu) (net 1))
 (segment (start 167.070379 72.451621) (end 169.084621 72.451621) (width 0.25) (layer F.Cu) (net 1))
 (segment (start 163.83 80.213131) (end 167.070379 72.451621) (width 0.25) (layer F.Cu) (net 1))
 (segment (start 169.084621 72.451621) (end 170.764 74.131) (width 0.25) (layer F.Cu) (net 1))
 (segment (start 163.83 86.207) (end 163.83 80.213131) (width 0.25) (layer F.Cu) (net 1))
 (segment (start 164.02 86.397) (end 163.83 86.207) (width 0.25) (layer F.Cu) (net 1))
 (segment (start 164.77 86.397) (end 164.02 86.397) (width 0.25) (layer F.Cu) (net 1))
 (segment (start 173.603872 77.970872) (end 173.685 78.165195) (width 0.25) (layer F.Cu) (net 1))
 (segment (start 170.764 75.131) (end 173.603872 77.970872) (width 0.25) (layer F.Cu) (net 1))
 (segment (start 173.685 78.165195) (end 173.685 81.497) (width 0.25) (layer F.Cu) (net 1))
 (segment (start 170.764 74.131) (end 170.764 75.131) (width 0.25) (layer F.Cu) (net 1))
 (segment (start 173.685 82.497) (end 176.733 85.545) (width 0.25) (layer F.Cu) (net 1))
 (segment (start 176.733 85.545) (end 176.733 88.863) (width 0.25) (layer F.Cu) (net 1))
 (segment (start 173.685 81.497) (end 173.685 82.497) (width 0.25) (layer F.Cu) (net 1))
 (segment (start 175.907999 94.773001) (end 175.907999 94.006999) (width 0.25) (layer F.Cu) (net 1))
 (segment (start 177.493001 94.838001) (end 175.972999 94.838001) (width 0.25) (layer F.Cu) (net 1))
 (segment (start 177.558001 94.773001) (end 177.493001 94.838001) (width 0.25) (layer F.Cu) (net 1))
 (segment (start 177.558001 90.688001) (end 177.558001 94.773001) (width 0.25) (layer F.Cu) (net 1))
 (segment (start 175.907999 94.006999) (end 170.764 88.863) (width 0.25) (layer F.Cu) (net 1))
 (segment (start 175.972999 94.838001) (end 175.907999 94.773001) (width 0.25) (layer F.Cu) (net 1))
 (segment (start 176.733 89.863) (end 177.558001 90.688001) (width 0.25) (layer F.Cu) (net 1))
 (segment (start 176.733 88.863) (end 176.733 89.863) (width 0.25) (layer F.Cu) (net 1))
 (segment (start 166.045011 83.421989) (end 167.97 81.497) (width 0.25) (layer F.Cu) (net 4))
 (segment (start 166.045011 87.612989) (end 166.045011 83.421989) (width 0.25) (layer F.Cu) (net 4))
 (segment (start 164.795 88.863) (end 166.045011 87.612989) (width 0.25) (layer F.Cu) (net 4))
 (segment (start 167.97 79.437) (end 167.564 79.031) (width 0.25) (layer F.Cu) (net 4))
 (segment (start 167.97 81.497) (end 167.97 79.437) (width 0.25) (layer F.Cu) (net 4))
 (segment (start 169.094001 87.787999) (end 170.485 86.397) (width 0.25) (layer F.Cu) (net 4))
 (segment (start 165.870001 87.787999) (end 169.094001 87.787999) (width 0.25) (layer F.Cu) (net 4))
 (segment (start 164.795 88.863) (end 165.870001 87.787999) (width 0.25) (layer F.Cu) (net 4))
 (segment (start 168.639001 94.838001) (end 167.564 93.763) (width 0.25) (layer F.Cu) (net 4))
 (segment (start 172.457999 94.838001) (end 168.639001 94.838001) (width 0.25) (layer F.Cu) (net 4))
 (segment (start 173.533 93.763) (end 172.457999 94.838001) (width 0.25) (layer F.Cu) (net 4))
 (segment (start 164.795 90.994) (end 167.564 93.763) (width 0.25) (layer F.Cu) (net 4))
 (segment (start 164.795 88.863) (end 164.795 90.994) (width 0.25) (layer F.Cu) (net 4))
 (segment (start 165.595001 87.407001) (end 165.595001 82.322001) (width 0.25) (layer F.Cu) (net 18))
 (segment (start 165.530001 87.472001) (end 165.595001 87.407001) (width 0.25) (layer F.Cu) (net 18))
 (segment (start 164.350997 87.472001) (end 165.530001 87.472001) (width 0.25) (layer F.Cu) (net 18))
 (segment (start 165.595001 82.322001) (end 164.77 81.497) (width 0.25) (layer F.Cu) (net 18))
 (segment (start 163.969999 87.852999) (end 164.350997 87.472001) (width 0.25) (layer F.Cu) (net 18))
 (segment (start 163.969999 92.937999) (end 163.969999 87.852999) (width 0.25) (layer F.Cu) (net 18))
 (segment (start 164.795 93.763) (end 163.969999 92.937999) (width 0.25) (layer F.Cu) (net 18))
 (segment (start 168.795001 80.999999) (end 170.764 79.031) (width 0.25) (layer F.Cu) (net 22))
 (segment (start 168.795001 85.571999) (end 168.795001 80.999999) (width 0.25) (layer F.Cu) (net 22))
 (segment (start 167.97 86.397) (end 168.795001 85.571999) (width 0.25) (layer F.Cu) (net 22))
 (segment (start 172.859999 85.571999) (end 173.685 86.397) (width 0.25) (layer F.Cu) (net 26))
 (segment (start 172.859999 78.676999) (end 172.859999 85.571999) (width 0.25) (layer F.Cu) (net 26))
 (segment (start 168.314 74.131) (end 172.859999 78.676999) (width 0.25) (layer F.Cu) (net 26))
 (segment (start 167.564 74.131) (end 168.314 74.131) (width 0.25) (layer F.Cu) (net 26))
 (segment (start 174.358001 91.388001) (end 176.733 93.763) (width 0.25) (layer F.Cu) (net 30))
 (segment (start 174.358001 87.852999) (end 174.358001 91.388001) (width 0.25) (layer F.Cu) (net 30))
 (segment (start 173.240997 87.787999) (end 174.293001 87.787999) (width 0.25) (layer F.Cu) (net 30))
 (segment (start 172.859999 86.208409) (end 172.859999 87.407001) (width 0.25) (layer F.Cu) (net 30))
 (segment (start 174.293001 87.787999) (end 174.358001 87.852999) (width 0.25) (layer F.Cu) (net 30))
 (segment (start 170.485 83.83341) (end 172.859999 86.208409) (width 0.25) (layer F.Cu) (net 30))
 (segment (start 172.859999 87.407001) (end 173.240997 87.787999) (width 0.25) (layer F.Cu) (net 30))
 (segment (start 170.485 81.497) (end 170.485 83.83341) (width 0.25) (layer F.Cu) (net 30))
 (segment (start 169.938999 92.937999) (end 170.764 93.763) (width 0.25) (layer F.Cu) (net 34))
 (segment (start 169.938999 87.852999) (end 169.938999 92.937999) (width 0.25) (layer F.Cu) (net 34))
 (segment (start 170.003999 87.787999) (end 169.938999 87.852999) (width 0.25) (layer F.Cu) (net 34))
 (segment (start 172.457999 87.787999) (end 170.003999 87.787999) (width 0.25) (layer F.Cu) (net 34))
 (segment (start 173.533 88.863) (end 172.457999 87.787999) (width 0.25) (layer F.Cu) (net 34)))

